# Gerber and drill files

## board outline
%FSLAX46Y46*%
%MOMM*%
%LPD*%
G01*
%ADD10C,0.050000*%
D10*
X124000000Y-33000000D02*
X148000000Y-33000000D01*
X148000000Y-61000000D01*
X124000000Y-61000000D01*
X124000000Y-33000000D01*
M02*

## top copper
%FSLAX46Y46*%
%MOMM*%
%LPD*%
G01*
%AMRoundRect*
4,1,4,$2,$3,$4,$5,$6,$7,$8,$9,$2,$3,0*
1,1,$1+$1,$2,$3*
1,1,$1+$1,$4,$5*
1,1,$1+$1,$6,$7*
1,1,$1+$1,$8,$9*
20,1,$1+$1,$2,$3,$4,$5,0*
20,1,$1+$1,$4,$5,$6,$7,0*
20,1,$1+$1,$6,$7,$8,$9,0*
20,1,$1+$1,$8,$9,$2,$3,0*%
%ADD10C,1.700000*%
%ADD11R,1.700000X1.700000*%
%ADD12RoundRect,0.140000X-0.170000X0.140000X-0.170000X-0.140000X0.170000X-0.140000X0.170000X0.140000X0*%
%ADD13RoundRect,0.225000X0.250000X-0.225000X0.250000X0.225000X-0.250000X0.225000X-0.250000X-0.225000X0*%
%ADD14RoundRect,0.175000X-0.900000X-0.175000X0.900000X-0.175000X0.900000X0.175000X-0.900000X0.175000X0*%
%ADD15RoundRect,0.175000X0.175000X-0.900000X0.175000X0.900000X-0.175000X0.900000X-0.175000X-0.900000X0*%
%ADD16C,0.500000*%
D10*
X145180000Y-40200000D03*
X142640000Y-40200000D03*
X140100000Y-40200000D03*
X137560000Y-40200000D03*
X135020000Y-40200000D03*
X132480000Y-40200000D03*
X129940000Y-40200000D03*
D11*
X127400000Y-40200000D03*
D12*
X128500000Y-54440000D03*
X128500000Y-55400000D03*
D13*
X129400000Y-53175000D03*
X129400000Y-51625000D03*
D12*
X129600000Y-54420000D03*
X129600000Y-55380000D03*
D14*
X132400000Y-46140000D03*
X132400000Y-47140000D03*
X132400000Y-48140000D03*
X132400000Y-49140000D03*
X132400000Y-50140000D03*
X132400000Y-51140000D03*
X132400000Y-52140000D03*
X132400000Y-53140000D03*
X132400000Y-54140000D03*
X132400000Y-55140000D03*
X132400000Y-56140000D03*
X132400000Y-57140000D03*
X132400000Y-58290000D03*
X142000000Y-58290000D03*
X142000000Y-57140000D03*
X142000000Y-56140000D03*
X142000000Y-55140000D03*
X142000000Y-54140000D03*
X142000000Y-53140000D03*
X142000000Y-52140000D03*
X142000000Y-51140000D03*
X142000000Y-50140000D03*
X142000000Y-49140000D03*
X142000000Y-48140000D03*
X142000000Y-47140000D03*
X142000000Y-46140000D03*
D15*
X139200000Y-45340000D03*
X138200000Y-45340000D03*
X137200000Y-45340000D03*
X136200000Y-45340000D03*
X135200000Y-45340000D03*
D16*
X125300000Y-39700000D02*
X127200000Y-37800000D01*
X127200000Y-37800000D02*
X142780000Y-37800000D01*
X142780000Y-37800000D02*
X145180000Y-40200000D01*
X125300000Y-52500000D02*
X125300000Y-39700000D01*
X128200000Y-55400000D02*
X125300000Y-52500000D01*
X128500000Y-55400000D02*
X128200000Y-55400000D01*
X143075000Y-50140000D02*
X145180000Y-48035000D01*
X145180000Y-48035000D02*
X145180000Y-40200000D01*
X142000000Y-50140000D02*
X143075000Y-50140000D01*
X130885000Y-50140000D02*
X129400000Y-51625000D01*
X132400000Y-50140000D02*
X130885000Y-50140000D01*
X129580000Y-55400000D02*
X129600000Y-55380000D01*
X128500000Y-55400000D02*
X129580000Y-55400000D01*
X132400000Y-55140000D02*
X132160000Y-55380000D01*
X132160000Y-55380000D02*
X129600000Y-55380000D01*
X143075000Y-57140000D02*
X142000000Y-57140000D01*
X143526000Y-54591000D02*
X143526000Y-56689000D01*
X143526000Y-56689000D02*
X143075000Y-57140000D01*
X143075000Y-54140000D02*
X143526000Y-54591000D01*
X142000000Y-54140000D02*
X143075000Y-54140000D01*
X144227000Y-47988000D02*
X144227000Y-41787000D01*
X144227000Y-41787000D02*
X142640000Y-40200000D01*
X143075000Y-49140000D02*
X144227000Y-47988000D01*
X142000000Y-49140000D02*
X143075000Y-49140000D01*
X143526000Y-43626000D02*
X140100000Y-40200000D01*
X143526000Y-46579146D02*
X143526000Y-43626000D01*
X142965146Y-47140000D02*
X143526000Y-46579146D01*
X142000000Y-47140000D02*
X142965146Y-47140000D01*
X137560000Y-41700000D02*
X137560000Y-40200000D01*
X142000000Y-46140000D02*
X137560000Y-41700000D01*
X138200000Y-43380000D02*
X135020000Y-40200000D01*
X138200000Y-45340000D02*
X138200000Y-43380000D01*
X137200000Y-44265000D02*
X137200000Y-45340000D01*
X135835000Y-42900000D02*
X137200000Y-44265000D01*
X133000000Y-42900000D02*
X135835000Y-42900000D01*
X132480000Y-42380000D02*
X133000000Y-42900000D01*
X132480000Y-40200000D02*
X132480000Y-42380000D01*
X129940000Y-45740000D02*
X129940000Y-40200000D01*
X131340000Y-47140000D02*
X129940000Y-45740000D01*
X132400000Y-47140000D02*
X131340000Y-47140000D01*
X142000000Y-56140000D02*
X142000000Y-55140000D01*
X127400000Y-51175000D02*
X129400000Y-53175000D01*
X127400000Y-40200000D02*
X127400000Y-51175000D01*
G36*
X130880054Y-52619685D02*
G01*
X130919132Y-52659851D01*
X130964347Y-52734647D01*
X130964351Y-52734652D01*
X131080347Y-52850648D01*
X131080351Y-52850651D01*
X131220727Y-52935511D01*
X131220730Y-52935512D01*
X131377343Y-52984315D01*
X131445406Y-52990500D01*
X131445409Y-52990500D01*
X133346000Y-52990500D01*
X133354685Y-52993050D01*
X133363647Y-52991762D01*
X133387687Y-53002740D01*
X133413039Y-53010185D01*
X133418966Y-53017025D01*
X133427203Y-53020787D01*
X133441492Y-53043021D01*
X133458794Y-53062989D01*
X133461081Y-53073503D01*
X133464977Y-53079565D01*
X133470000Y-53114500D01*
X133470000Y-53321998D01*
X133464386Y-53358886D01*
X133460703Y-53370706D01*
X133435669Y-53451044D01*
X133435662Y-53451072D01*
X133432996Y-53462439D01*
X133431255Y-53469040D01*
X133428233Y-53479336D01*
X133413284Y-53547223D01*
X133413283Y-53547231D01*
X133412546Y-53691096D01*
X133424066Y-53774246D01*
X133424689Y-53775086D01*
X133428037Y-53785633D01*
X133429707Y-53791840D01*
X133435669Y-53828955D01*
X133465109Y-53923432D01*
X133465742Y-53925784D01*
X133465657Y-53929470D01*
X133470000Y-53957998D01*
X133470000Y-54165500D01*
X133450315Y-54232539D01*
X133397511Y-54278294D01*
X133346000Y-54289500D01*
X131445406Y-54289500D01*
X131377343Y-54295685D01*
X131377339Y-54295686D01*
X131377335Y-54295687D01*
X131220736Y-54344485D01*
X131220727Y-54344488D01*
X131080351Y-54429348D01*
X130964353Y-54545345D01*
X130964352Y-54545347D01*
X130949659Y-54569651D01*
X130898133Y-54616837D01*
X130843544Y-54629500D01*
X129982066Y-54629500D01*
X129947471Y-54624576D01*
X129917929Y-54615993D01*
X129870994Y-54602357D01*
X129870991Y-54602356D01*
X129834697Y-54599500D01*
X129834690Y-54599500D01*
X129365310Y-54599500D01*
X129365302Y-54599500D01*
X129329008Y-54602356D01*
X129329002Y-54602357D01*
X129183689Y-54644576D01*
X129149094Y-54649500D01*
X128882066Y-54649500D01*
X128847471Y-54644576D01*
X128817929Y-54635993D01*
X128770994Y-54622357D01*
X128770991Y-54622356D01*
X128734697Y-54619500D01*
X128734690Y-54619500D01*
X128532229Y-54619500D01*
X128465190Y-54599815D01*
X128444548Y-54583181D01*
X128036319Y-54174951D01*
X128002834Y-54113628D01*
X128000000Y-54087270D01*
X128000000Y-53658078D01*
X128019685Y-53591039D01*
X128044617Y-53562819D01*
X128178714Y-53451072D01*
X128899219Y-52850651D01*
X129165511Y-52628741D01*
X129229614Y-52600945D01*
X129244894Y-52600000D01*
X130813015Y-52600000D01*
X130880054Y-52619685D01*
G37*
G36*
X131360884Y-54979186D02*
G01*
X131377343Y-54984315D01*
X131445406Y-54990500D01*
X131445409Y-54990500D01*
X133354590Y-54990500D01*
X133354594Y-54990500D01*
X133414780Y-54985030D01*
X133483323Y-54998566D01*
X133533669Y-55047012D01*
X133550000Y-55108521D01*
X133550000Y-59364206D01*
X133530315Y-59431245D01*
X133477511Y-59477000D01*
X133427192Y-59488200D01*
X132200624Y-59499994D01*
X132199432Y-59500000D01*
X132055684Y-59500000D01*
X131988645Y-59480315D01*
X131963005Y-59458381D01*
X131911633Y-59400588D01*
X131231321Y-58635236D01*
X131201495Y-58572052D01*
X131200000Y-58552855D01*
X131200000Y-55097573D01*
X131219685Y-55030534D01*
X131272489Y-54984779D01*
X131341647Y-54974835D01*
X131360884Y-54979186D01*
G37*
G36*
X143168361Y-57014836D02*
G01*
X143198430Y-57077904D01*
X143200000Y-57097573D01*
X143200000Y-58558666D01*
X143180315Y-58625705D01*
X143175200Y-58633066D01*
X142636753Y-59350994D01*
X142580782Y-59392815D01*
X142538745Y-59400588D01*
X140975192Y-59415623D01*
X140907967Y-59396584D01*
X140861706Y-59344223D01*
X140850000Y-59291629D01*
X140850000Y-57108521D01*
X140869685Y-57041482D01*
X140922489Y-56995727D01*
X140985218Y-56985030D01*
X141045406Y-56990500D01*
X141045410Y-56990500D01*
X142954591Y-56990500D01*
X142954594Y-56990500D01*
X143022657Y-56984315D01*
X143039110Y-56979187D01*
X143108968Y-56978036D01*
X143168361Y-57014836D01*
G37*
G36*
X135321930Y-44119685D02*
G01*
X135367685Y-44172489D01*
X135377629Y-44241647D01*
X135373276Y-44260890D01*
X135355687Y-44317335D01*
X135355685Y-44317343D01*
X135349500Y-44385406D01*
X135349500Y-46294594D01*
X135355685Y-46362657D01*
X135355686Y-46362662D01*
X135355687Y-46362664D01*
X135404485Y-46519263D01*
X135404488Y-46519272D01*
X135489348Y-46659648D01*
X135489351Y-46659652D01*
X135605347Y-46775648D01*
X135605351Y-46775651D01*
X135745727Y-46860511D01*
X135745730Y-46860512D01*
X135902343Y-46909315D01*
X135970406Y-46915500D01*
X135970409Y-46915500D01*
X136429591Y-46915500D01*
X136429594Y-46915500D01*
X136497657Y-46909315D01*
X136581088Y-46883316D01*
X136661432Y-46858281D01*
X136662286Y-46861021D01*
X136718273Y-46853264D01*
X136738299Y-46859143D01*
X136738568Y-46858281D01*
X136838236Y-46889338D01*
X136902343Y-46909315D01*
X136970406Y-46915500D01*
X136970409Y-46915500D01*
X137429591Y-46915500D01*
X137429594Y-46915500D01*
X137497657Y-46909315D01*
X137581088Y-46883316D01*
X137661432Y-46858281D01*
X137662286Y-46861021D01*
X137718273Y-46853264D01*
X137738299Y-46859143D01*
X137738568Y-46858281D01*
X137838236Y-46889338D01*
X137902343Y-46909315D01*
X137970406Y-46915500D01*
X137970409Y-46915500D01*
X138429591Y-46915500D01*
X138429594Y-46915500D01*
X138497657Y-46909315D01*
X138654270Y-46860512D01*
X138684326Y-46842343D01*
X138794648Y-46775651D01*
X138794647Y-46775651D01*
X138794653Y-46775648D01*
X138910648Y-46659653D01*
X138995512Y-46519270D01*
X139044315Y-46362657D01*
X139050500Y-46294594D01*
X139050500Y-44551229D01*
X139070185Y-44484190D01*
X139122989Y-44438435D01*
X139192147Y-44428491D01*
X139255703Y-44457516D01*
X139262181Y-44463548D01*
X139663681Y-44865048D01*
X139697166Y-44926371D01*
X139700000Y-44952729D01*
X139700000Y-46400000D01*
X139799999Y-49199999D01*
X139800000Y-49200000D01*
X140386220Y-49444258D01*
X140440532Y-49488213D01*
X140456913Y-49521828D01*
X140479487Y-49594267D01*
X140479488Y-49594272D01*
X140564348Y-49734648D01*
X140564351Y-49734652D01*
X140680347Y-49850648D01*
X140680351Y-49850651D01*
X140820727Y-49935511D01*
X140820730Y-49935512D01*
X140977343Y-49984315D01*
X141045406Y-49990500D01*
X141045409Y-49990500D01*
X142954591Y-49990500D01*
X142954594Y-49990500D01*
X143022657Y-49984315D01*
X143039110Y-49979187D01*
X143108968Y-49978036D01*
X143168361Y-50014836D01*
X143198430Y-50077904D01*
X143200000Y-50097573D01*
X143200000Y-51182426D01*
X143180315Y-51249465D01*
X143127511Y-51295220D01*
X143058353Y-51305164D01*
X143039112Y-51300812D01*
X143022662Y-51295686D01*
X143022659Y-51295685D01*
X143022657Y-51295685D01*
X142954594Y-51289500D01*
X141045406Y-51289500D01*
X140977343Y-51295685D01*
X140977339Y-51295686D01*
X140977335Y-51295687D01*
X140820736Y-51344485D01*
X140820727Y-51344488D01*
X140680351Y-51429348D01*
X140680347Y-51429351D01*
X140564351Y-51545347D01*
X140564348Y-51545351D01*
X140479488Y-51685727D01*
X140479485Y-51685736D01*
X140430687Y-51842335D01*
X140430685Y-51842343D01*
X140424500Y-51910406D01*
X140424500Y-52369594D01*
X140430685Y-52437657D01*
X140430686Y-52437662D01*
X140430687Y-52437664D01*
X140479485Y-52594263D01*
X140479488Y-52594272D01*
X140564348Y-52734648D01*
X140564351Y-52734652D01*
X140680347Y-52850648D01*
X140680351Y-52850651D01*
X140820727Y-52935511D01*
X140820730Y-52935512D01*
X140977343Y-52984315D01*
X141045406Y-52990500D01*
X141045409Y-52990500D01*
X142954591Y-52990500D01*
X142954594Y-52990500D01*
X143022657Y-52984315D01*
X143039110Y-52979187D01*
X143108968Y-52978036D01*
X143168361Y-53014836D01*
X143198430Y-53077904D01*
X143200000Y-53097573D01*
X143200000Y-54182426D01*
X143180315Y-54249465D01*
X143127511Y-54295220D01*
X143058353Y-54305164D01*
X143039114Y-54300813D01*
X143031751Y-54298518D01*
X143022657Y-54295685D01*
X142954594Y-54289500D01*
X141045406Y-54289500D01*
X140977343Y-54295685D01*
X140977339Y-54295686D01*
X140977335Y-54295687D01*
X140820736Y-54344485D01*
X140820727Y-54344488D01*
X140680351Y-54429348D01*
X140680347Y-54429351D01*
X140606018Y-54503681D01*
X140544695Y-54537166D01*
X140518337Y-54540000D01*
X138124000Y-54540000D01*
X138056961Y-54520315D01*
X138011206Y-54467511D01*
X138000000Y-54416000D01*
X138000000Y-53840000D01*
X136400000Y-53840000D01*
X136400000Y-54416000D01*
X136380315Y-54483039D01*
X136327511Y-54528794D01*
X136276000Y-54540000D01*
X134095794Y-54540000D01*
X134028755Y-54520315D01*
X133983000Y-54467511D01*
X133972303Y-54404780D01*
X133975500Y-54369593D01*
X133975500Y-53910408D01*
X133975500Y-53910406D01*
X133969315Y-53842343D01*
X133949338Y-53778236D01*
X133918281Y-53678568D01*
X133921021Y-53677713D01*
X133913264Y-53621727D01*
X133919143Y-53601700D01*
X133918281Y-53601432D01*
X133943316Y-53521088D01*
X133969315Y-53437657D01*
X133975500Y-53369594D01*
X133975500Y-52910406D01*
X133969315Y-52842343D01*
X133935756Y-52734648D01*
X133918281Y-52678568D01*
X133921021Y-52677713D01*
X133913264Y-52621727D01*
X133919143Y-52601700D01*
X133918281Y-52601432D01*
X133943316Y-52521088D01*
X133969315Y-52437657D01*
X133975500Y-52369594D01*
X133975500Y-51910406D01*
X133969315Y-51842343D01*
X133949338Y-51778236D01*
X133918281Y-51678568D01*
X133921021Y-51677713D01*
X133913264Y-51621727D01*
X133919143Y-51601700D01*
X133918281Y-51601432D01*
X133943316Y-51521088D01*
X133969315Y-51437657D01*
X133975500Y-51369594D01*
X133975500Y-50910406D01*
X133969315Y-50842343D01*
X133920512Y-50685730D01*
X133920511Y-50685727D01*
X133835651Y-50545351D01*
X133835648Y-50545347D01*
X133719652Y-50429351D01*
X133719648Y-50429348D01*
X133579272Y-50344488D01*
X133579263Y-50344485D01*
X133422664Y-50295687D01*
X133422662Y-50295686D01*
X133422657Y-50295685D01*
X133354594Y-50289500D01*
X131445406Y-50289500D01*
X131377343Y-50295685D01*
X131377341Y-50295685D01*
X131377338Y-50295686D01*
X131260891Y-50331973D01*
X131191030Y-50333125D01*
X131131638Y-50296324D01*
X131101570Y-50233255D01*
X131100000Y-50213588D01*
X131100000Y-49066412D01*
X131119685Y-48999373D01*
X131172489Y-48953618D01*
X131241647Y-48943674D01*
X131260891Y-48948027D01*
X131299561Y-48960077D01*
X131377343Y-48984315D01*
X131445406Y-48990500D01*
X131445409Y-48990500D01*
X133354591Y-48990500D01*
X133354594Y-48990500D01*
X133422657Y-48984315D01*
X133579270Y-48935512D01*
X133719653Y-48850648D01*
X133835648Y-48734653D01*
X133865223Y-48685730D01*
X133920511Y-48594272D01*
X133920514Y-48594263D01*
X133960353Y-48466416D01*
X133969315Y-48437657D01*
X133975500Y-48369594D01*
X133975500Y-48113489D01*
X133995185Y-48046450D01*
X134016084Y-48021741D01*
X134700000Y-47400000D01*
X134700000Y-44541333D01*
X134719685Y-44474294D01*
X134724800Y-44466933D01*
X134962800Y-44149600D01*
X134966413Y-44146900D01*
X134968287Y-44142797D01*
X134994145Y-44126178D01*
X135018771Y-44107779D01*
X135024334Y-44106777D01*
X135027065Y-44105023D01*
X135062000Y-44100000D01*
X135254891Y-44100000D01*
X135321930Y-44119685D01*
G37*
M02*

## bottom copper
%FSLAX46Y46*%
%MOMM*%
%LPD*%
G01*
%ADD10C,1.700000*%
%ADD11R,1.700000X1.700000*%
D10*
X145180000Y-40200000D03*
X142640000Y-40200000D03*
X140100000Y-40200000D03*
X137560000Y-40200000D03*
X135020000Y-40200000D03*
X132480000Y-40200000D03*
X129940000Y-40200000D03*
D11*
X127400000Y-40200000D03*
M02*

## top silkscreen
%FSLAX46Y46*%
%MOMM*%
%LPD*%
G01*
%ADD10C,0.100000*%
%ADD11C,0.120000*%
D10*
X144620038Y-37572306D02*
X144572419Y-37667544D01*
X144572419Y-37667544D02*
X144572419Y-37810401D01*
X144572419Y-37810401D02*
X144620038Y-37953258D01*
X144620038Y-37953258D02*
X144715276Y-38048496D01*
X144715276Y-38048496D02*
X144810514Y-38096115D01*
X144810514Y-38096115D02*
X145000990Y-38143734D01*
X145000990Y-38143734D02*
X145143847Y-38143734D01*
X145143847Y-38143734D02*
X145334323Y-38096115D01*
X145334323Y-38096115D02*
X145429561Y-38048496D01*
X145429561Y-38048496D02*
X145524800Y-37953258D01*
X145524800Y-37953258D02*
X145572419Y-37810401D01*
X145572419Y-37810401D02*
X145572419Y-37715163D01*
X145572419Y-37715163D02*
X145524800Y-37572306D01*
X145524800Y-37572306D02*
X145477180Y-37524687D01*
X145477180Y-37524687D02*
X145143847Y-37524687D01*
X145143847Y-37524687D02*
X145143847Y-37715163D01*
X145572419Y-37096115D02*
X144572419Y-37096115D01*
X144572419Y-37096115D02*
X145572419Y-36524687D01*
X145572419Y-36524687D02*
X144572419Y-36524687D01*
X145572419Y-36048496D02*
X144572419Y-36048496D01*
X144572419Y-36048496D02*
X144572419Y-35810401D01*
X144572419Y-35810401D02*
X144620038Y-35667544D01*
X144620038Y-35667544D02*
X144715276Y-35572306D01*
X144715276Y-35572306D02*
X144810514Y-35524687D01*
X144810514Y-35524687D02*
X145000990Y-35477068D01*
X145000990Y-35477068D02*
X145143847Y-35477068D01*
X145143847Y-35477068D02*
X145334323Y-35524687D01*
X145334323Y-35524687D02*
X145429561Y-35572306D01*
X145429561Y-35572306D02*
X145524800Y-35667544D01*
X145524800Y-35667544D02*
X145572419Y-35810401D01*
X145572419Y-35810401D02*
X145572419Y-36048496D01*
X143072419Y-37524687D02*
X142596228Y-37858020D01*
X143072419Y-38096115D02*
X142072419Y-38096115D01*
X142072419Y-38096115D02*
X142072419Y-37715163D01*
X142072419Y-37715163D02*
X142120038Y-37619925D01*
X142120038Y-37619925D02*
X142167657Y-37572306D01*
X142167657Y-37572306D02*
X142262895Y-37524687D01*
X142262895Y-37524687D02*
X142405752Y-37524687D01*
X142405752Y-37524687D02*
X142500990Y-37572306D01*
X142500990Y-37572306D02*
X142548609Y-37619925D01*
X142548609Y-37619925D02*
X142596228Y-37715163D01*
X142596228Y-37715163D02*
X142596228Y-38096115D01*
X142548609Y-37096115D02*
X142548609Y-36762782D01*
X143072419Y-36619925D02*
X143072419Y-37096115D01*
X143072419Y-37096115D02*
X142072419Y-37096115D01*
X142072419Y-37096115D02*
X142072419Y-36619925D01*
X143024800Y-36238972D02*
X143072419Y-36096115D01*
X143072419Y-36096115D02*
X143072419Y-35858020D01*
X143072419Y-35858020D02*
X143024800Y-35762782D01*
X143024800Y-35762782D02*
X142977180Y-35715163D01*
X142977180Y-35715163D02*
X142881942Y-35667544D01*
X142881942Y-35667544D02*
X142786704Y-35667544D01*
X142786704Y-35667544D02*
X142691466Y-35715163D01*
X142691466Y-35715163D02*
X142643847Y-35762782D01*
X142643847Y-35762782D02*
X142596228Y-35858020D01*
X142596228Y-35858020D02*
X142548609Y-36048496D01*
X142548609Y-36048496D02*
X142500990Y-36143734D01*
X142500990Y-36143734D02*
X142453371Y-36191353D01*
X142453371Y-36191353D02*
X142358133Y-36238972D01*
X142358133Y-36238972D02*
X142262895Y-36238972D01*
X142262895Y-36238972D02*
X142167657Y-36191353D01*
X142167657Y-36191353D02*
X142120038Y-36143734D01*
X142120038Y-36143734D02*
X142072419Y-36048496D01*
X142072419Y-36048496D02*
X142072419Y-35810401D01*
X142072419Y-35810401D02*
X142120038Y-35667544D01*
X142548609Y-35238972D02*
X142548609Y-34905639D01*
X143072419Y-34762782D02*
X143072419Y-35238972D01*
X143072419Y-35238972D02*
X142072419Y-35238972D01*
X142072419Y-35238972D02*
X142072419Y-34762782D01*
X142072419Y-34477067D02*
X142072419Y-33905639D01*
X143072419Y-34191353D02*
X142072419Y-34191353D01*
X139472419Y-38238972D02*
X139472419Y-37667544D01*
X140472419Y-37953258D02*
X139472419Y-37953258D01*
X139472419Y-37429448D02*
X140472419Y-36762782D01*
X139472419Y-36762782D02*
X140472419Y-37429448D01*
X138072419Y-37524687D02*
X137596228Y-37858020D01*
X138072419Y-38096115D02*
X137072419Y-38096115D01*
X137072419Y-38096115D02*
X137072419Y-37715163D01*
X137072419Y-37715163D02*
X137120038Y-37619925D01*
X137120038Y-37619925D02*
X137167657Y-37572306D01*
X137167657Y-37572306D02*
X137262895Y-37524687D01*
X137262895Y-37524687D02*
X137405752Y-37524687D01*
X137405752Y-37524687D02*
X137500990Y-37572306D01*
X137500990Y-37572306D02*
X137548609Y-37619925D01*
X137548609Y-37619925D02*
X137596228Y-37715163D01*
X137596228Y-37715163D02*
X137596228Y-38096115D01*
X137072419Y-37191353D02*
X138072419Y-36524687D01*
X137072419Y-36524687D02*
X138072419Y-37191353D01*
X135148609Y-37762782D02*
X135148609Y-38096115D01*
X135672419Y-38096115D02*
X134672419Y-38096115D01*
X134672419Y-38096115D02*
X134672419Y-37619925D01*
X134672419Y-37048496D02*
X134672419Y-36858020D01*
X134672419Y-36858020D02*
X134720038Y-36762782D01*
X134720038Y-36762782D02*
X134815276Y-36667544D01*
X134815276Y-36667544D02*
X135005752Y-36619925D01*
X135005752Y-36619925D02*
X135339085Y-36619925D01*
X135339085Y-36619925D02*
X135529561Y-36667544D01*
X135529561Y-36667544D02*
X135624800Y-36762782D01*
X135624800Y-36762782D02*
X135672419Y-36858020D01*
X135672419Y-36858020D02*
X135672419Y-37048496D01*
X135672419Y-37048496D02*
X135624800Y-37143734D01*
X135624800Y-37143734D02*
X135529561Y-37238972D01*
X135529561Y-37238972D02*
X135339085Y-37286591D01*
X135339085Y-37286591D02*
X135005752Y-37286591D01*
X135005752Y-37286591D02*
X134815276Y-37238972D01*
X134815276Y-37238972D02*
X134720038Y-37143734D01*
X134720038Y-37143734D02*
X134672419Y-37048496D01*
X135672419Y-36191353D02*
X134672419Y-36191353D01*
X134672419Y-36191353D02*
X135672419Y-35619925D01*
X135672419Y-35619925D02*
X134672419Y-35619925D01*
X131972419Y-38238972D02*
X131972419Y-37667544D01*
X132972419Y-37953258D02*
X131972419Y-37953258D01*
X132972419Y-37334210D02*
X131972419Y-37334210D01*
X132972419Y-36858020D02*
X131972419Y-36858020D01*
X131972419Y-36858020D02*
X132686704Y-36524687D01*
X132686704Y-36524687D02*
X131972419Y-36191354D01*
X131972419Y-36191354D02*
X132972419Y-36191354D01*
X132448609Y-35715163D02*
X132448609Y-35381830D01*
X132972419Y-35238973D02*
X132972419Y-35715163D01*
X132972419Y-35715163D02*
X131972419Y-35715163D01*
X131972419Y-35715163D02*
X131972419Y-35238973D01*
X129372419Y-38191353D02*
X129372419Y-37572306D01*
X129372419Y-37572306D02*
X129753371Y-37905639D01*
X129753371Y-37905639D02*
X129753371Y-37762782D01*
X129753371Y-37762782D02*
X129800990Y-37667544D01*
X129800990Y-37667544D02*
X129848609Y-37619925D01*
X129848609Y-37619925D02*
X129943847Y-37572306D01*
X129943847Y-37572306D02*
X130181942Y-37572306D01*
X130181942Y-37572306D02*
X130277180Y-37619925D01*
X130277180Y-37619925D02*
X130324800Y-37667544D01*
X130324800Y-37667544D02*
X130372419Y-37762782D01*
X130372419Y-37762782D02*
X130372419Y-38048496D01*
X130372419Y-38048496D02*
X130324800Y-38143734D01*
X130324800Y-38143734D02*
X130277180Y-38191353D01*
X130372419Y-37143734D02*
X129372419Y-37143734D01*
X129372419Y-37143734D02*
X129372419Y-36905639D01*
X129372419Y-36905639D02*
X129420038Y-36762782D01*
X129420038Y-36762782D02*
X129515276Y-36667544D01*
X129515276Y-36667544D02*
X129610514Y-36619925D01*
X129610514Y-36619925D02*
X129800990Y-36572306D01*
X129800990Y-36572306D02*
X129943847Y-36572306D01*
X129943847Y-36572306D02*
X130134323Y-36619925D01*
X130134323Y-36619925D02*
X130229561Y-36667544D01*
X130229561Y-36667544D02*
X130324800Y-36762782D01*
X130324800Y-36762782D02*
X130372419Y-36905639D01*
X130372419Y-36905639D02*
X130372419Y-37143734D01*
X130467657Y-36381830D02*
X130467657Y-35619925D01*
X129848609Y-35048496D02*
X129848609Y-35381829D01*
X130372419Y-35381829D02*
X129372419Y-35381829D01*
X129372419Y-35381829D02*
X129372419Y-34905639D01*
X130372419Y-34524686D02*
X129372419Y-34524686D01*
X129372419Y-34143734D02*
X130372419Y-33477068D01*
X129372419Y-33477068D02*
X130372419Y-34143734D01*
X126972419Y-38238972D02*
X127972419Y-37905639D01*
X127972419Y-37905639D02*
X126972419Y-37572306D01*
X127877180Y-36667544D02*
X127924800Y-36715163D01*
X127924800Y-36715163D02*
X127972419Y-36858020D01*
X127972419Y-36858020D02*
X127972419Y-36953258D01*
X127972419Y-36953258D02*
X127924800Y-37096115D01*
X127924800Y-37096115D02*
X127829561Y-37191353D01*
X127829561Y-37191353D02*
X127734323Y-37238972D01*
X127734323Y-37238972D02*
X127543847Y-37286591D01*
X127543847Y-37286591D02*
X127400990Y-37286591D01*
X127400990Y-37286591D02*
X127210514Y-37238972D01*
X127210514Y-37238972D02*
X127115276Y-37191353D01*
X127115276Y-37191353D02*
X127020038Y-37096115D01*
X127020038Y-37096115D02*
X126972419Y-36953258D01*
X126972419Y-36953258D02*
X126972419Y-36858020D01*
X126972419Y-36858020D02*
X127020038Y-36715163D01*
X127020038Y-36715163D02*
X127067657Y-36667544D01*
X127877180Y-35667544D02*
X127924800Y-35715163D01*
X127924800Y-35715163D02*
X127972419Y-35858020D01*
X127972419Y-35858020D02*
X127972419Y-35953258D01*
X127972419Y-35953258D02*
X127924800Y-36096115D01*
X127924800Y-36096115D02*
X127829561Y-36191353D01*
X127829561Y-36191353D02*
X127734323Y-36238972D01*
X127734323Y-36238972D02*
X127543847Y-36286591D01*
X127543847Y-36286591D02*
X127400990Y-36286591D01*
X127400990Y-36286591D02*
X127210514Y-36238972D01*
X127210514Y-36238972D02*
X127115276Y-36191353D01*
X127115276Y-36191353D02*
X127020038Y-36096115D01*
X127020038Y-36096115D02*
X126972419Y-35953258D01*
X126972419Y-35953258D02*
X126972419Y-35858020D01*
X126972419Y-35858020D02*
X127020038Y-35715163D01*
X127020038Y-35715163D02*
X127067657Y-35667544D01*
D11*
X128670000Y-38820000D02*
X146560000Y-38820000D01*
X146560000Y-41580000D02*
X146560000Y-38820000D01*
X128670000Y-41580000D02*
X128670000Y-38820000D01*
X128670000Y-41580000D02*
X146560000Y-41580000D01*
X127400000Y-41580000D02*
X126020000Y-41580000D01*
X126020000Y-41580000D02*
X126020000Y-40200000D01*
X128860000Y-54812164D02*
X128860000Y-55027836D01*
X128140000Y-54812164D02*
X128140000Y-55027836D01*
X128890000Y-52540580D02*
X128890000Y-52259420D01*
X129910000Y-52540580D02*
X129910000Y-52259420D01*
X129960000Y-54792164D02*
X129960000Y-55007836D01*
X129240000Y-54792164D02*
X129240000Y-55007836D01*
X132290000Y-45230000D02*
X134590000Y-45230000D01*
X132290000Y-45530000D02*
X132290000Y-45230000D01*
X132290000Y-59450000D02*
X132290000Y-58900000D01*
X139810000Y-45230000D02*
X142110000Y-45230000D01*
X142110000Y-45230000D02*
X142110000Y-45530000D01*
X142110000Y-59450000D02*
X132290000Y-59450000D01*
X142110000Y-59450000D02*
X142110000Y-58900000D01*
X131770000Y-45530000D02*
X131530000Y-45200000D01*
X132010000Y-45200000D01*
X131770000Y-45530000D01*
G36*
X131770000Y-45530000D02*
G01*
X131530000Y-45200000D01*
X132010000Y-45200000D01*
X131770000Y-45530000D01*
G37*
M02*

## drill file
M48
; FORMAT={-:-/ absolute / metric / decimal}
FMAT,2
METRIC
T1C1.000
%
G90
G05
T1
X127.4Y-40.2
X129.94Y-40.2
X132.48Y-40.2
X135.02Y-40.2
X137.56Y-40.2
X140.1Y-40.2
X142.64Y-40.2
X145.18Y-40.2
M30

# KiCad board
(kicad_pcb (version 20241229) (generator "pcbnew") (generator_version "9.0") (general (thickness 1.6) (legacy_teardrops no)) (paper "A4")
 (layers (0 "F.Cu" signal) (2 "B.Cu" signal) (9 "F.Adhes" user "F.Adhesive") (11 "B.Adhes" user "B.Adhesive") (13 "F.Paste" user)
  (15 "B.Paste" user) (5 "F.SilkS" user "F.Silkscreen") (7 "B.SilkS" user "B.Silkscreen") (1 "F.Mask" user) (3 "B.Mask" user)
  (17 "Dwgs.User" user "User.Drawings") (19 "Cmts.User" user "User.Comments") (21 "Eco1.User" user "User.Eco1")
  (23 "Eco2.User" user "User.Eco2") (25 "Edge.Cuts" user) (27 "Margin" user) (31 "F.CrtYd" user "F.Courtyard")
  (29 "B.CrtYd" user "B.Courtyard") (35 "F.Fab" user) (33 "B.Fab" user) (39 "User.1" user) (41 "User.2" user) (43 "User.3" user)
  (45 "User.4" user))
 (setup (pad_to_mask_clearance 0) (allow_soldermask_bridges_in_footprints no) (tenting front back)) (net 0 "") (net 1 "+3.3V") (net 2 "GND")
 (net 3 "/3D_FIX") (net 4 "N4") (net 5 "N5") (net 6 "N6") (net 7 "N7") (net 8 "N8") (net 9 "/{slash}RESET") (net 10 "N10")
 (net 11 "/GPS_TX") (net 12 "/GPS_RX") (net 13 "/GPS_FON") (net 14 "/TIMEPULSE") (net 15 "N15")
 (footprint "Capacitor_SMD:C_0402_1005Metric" (layer "F.Cu") (at 128.5 54.92 -90)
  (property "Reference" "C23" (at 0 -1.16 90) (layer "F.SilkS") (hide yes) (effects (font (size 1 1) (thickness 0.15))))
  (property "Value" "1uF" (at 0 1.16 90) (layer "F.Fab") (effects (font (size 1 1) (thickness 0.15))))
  (fp_line (start -0.107836 0.36) (end 0.107836 0.36) (stroke (width 0.12) (type solid)) (layer "F.SilkS"))
  (fp_line (start -0.107836 -0.36) (end 0.107836 -0.36) (stroke (width 0.12) (type solid)) (layer "F.SilkS"))
  (pad "1" smd roundrect (at -0.48 0 270) (size 0.56 0.62) (layers "F.Cu" "F.Mask" "F.Paste") (roundrect_rratio 0.25) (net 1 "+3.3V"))
  (pad "2" smd roundrect (at 0.48 0 270) (size 0.56 0.62) (layers "F.Cu" "F.Mask" "F.Paste") (roundrect_rratio 0.25) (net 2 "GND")))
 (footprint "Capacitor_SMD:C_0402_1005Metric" (layer "F.Cu") (at 129.6 54.9 -90)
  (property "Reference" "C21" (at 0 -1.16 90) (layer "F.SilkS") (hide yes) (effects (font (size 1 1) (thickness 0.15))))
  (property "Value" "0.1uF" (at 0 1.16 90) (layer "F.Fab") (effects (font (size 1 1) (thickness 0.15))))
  (fp_line (start -0.107836 0.36) (end 0.107836 0.36) (stroke (width 0.12) (type solid)) (layer "F.SilkS"))
  (fp_line (start -0.107836 -0.36) (end 0.107836 -0.36) (stroke (width 0.12) (type solid)) (layer "F.SilkS"))
  (pad "1" smd roundrect (at -0.48 0 270) (size 0.56 0.62) (layers "F.Cu" "F.Mask" "F.Paste") (roundrect_rratio 0.25) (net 1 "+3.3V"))
  (pad "2" smd roundrect (at 0.48 0 270) (size 0.56 0.62) (layers "F.Cu" "F.Mask" "F.Paste") (roundrect_rratio 0.25) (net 2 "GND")))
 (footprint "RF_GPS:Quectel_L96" (layer "F.Cu") (at 137.2 52.34)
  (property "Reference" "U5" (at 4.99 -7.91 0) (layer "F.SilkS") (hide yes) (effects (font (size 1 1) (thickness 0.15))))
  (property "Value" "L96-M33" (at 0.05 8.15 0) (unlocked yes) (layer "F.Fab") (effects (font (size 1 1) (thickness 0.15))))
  (fp_line (start -4.91 -7.11) (end -2.61 -7.11) (stroke (width 0.12) (type default)) (layer "F.SilkS"))
  (fp_line (start -4.91 -6.81) (end -4.91 -7.11) (stroke (width 0.12) (type default)) (layer "F.SilkS"))
  (fp_line (start -4.91 7.11) (end -4.91 6.56) (stroke (width 0.12) (type default)) (layer "F.SilkS"))
  (fp_line (start 2.61 -7.11) (end 4.91 -7.11) (stroke (width 0.12) (type default)) (layer "F.SilkS"))
  (fp_line (start 4.91 -7.11) (end 4.91 -6.81) (stroke (width 0.12) (type default)) (layer "F.SilkS"))
  (fp_line (start 4.91 7.11) (end -4.91 7.11) (stroke (width 0.12) (type default)) (layer "F.SilkS"))
  (fp_line (start 4.91 7.11) (end 4.91 6.56) (stroke (width 0.12) (type default)) (layer "F.SilkS"))
  (fp_poly
   (pts (xy -5.43 -6.81) (xy -5.67 -7.14) (xy -5.19 -7.14) (xy -5.43 -6.81)) (stroke (width 0.12) (type solid)) (fill yes) (layer "F.SilkS"))
  (pad "1" smd roundrect (at -4.8 -6.2) (size 2.15 0.7) (layers "F.Cu" "F.Mask" "F.Paste") (roundrect_rratio 0.25) (thermal_bridge_angle 45))
  (pad "2" smd roundrect (at -4.8 -5.2) (size 2.15 0.7) (layers "F.Cu" "F.Mask" "F.Paste") (roundrect_rratio 0.25) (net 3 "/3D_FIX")
   (thermal_bridge_angle 45))
  (pad "3" smd roundrect (at -4.8 -4.2) (size 2.15 0.7) (layers "F.Cu" "F.Mask" "F.Paste") (roundrect_rratio 0.25) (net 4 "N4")
   (thermal_bridge_angle 45))
  (pad "4" smd roundrect (at -4.8 -3.2) (size 2.15 0.7) (layers "F.Cu" "F.Mask" "F.Paste") (roundrect_rratio 0.25) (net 2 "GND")
   (thermal_bridge_angle 45))
  (pad "5" smd roundrect (at -4.8 -2.2) (size 2.15 0.7) (layers "F.Cu" "F.Mask" "F.Paste") (roundrect_rratio 0.25) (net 2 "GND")
   (thermal_bridge_angle 45))
  (pad "6" smd roundrect (at -4.8 -1.2) (size 2.15 0.7) (layers "F.Cu" "F.Mask" "F.Paste") (roundrect_rratio 0.25) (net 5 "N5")
   (thermal_bridge_angle 45))
  (pad "7" smd roundrect (at -4.8 -0.2) (size 2.15 0.7) (layers "F.Cu" "F.Mask" "F.Paste") (roundrect_rratio 0.25) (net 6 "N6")
   (thermal_bridge_angle 45))
  (pad "8" smd roundrect (at -4.8 0.8) (size 2.15 0.7) (layers "F.Cu" "F.Mask" "F.Paste") (roundrect_rratio 0.25) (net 1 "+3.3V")
   (thermal_bridge_angle 45))
  (pad "9" smd roundrect (at -4.8 1.8) (size 2.15 0.7) (layers "F.Cu" "F.Mask" "F.Paste") (roundrect_rratio 0.25) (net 1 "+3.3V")
   (thermal_bridge_angle 45))
  (pad "10" smd roundrect (at -4.8 2.8) (size 2.15 0.7) (layers "F.Cu" "F.Mask" "F.Paste") (roundrect_rratio 0.25) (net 2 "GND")
   (thermal_bridge_angle 45))
  (pad "11" smd roundrect (at -4.8 3.8) (size 2.15 0.7) (layers "F.Cu" "F.Mask" "F.Paste") (roundrect_rratio 0.25) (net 2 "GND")
   (thermal_bridge_angle 45))
  (pad "12" smd roundrect (at -4.8 4.8) (size 2.15 0.7) (layers "F.Cu" "F.Mask" "F.Paste") (roundrect_rratio 0.25) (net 2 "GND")
   (thermal_bridge_angle 45))
  (pad "13" smd roundrect (at -4.8 5.95) (size 2.15 0.7) (layers "F.Cu" "F.Mask" "F.Paste") (roundrect_rratio 0.25) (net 2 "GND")
   (thermal_bridge_angle 45))
  (pad "14" smd roundrect (at 4.8 5.95) (size 2.15 0.7) (layers "F.Cu" "F.Mask" "F.Paste") (roundrect_rratio 0.25) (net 2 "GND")
   (thermal_bridge_angle 45))
  (pad "15" smd roundrect (at 4.8 4.8) (size 2.15 0.7) (layers "F.Cu" "F.Mask" "F.Paste") (roundrect_rratio 0.25) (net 2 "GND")
   (thermal_bridge_angle 45))
  (pad "16" smd roundrect (at 4.8 3.8) (size 2.15 0.7) (layers "F.Cu" "F.Mask" "F.Paste") (roundrect_rratio 0.25) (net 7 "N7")
   (thermal_bridge_angle 45))
  (pad "17" smd roundrect (at 4.8 2.8) (size 2.15 0.7) (layers "F.Cu" "F.Mask" "F.Paste") (roundrect_rratio 0.25) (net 7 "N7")
   (thermal_bridge_angle 45))
  (pad "18" smd roundrect (at 4.8 1.8) (size 2.15 0.7) (layers "F.Cu" "F.Mask" "F.Paste") (roundrect_rratio 0.25) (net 2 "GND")
   (thermal_bridge_angle 45))
  (pad "19" smd roundrect (at 4.8 0.8) (size 2.15 0.7) (layers "F.Cu" "F.Mask" "F.Paste") (roundrect_rratio 0.25) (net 2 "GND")
   (thermal_bridge_angle 45))
  (pad "20" smd roundrect (at 4.8 -0.2) (size 2.15 0.7) (layers "F.Cu" "F.Mask" "F.Paste") (roundrect_rratio 0.25) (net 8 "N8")
   (thermal_bridge_angle 45))
  (pad "21" smd roundrect (at 4.8 -1.2) (size 2.15 0.7) (layers "F.Cu" "F.Mask" "F.Paste") (roundrect_rratio 0.25) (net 2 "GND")
   (thermal_bridge_angle 45))
  (pad "22" smd roundrect (at 4.8 -2.2) (size 2.15 0.7) (layers "F.Cu" "F.Mask" "F.Paste") (roundrect_rratio 0.25) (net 2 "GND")
   (thermal_bridge_angle 45))
  (pad "23" smd roundrect (at 4.8 -3.2) (size 2.15 0.7) (layers "F.Cu" "F.Mask" "F.Paste") (roundrect_rratio 0.25) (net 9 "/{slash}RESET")
   (thermal_bridge_angle 45))
  (pad "24" smd roundrect (at 4.8 -4.2) (size 2.15 0.7) (layers "F.Cu" "F.Mask" "F.Paste") (roundrect_rratio 0.25) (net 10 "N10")
   (thermal_bridge_angle 45))
  (pad "25" smd roundrect (at 4.8 -5.2) (size 2.15 0.7) (layers "F.Cu" "F.Mask" "F.Paste") (roundrect_rratio 0.25) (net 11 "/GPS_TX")
   (thermal_bridge_angle 45))
  (pad "26" smd roundrect (at 4.8 -6.2) (size 2.15 0.7) (layers "F.Cu" "F.Mask" "F.Paste") (roundrect_rratio 0.25) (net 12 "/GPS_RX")
   (thermal_bridge_angle 45))
  (pad "27" smd roundrect (at 2 -7 90) (size 2.15 0.7) (layers "F.Cu" "F.Mask" "F.Paste") (roundrect_rratio 0.25) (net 2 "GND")
   (thermal_bridge_angle 45))
  (pad "28" smd roundrect (at 1 -7 90) (size 2.15 0.7) (layers "F.Cu" "F.Mask" "F.Paste") (roundrect_rratio 0.25) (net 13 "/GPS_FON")
   (thermal_bridge_angle 45))
  (pad "29" smd roundrect (at 0 -7 90) (size 2.15 0.7) (layers "F.Cu" "F.Mask" "F.Paste") (roundrect_rratio 0.25) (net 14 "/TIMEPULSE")
   (thermal_bridge_angle 45))
  (pad "30" smd roundrect (at -1 -7 90) (size 2.15 0.7) (layers "F.Cu" "F.Mask" "F.Paste") (roundrect_rratio 0.25) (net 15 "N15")
   (thermal_bridge_angle 45))
  (pad "31" smd roundrect (at -2 -7 90) (size 2.15 0.7) (layers "F.Cu" "F.Mask" "F.Paste") (roundrect_rratio 0.25) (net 2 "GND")
   (thermal_bridge_angle 45))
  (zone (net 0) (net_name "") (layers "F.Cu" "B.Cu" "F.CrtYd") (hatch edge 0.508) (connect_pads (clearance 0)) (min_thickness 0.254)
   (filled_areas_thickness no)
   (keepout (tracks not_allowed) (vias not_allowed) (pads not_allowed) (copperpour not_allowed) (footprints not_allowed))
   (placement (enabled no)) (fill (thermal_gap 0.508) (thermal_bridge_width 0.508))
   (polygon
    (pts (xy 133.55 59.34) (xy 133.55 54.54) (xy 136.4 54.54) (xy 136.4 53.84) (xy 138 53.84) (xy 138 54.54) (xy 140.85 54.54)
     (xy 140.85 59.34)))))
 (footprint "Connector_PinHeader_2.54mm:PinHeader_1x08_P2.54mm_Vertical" (layer "F.Cu") (at 127.4 40.2 90)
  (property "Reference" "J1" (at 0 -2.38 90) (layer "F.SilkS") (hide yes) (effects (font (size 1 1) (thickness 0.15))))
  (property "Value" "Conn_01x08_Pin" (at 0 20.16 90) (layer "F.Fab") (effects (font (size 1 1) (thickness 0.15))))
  (fp_line (start -1.38 -1.38) (end 0 -1.38) (stroke (width 0.12) (type solid)) (layer "F.SilkS"))
  (fp_line (start -1.38 0) (end -1.38 -1.38) (stroke (width 0.12) (type solid)) (layer "F.SilkS"))
  (fp_line (start 1.38 1.27) (end 1.38 19.16) (stroke (width 0.12) (type solid)) (layer "F.SilkS"))
  (fp_line (start -1.38 1.27) (end 1.38 1.27) (stroke (width 0.12) (type solid)) (layer "F.SilkS"))
  (fp_line (start -1.38 1.27) (end -1.38 19.16) (stroke (width 0.12) (type solid)) (layer "F.SilkS"))
  (fp_line (start -1.38 19.16) (end 1.38 19.16) (stroke (width 0.12) (type solid)) (layer "F.SilkS"))
  (pad "1" thru_hole rect (at 0 0 90) (size 1.7 1.7) (drill 1) (layers "*.Cu" "*.Mask") (remove_unused_layers no) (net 1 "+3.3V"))
  (pad "2" thru_hole circle (at 0 2.54 90) (size 1.7 1.7) (drill 1) (layers "*.Cu" "*.Mask") (remove_unused_layers no) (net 3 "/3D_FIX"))
  (pad "3" thru_hole circle (at 0 5.08 90) (size 1.7 1.7) (drill 1) (layers "*.Cu" "*.Mask") (remove_unused_layers no) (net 14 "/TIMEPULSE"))
  (pad "4" thru_hole circle (at 0 7.62 90) (size 1.7 1.7) (drill 1) (layers "*.Cu" "*.Mask") (remove_unused_layers no) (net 13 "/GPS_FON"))
  (pad "5" thru_hole circle (at 0 10.16 90) (size 1.7 1.7) (drill 1) (layers "*.Cu" "*.Mask") (remove_unused_layers no) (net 12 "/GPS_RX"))
  (pad "6" thru_hole circle (at 0 12.7 90) (size 1.7 1.7) (drill 1) (layers "*.Cu" "*.Mask") (remove_unused_layers no) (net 11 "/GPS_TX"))
  (pad "7" thru_hole circle (at 0 15.24 90) (size 1.7 1.7) (drill 1) (layers "*.Cu" "*.Mask") (remove_unused_layers no)
   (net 9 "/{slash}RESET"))
  (pad "8" thru_hole circle (at 0 17.78 90) (size 1.7 1.7) (drill 1) (layers "*.Cu" "*.Mask") (remove_unused_layers no) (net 2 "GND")))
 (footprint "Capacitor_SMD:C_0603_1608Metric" (layer "F.Cu") (at 129.4 52.4 90)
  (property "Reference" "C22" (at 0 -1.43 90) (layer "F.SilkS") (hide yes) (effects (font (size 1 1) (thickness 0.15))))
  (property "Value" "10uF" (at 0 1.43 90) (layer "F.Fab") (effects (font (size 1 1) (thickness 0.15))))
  (fp_line (start -0.14058 -0.51) (end 0.14058 -0.51) (stroke (width 0.12) (type solid)) (layer "F.SilkS"))
  (fp_line (start -0.14058 0.51) (end 0.14058 0.51) (stroke (width 0.12) (type solid)) (layer "F.SilkS"))
  (pad "1" smd roundrect (at -0.775 0 90) (size 0.9 0.95) (layers "F.Cu" "F.Mask" "F.Paste") (roundrect_rratio 0.25) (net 1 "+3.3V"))
  (pad "2" smd roundrect (at 0.775 0 90) (size 0.9 0.95) (layers "F.Cu" "F.Mask" "F.Paste") (roundrect_rratio 0.25) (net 2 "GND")))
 (gr_rect (start 124 33) (end 148 61) (stroke (width 0.05) (type default)) (fill no) (layer "Edge.Cuts"))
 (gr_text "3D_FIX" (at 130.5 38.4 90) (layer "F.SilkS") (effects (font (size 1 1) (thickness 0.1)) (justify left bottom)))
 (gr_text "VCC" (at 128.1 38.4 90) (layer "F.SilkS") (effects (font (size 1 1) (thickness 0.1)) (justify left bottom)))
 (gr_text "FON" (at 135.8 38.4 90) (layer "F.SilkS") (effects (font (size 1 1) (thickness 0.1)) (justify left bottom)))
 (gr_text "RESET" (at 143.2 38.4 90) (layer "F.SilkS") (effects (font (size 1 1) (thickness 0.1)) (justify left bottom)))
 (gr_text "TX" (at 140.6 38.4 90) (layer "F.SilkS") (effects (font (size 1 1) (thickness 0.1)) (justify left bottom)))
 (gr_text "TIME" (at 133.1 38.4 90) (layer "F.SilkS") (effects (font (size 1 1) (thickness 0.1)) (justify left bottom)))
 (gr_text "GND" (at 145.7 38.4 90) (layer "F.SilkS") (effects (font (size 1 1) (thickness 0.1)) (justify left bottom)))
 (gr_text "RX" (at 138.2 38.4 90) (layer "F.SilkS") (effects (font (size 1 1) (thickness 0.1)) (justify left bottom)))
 (segment (start 143.075 50.14) (end 145.18 48.035) (width 0.5) (layer "F.Cu") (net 2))
 (segment (start 143.075 54.14) (end 143.526 54.591) (width 0.5) (layer "F.Cu") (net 2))
 (segment (start 143.075 57.14) (end 142 57.14) (width 0.5) (layer "F.Cu") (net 2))
 (segment (start 130.885 50.14) (end 129.4 51.625) (width 0.5) (layer "F.Cu") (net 2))
 (segment (start 128.5 55.4) (end 128.2 55.4) (width 0.5) (layer "F.Cu") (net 2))
 (segment (start 125.3 39.7) (end 127.2 37.8) (width 0.5) (layer "F.Cu") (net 2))
 (segment (start 142 50.14) (end 143.075 50.14) (width 0.5) (layer "F.Cu") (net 2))
 (segment (start 128.5 55.4) (end 129.58 55.4) (width 0.5) (layer "F.Cu") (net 2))
 (segment (start 128.2 55.4) (end 125.3 52.5) (width 0.5) (layer "F.Cu") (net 2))
 (segment (start 132.4 50.14) (end 130.885 50.14) (width 0.5) (layer "F.Cu") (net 2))
 (segment (start 129.58 55.4) (end 129.6 55.38) (width 0.5) (layer "F.Cu") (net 2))
 (segment (start 142.78 37.8) (end 145.18 40.2) (width 0.5) (layer "F.Cu") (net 2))
 (segment (start 142 54.14) (end 143.075 54.14) (width 0.5) (layer "F.Cu") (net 2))
 (segment (start 143.526 56.689) (end 143.075 57.14) (width 0.5) (layer "F.Cu") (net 2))
 (segment (start 145.18 48.035) (end 145.18 40.2) (width 0.5) (layer "F.Cu") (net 2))
 (segment (start 125.3 52.5) (end 125.3 39.7) (width 0.5) (layer "F.Cu") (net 2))
 (segment (start 127.2 37.8) (end 142.78 37.8) (width 0.5) (layer "F.Cu") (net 2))
 (segment (start 143.526 54.591) (end 143.526 56.689) (width 0.5) (layer "F.Cu") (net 2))
 (segment (start 132.16 55.38) (end 129.6 55.38) (width 0.5) (layer "F.Cu") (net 2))
 (segment (start 132.4 55.14) (end 132.16 55.38) (width 0.5) (layer "F.Cu") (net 2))
 (segment (start 127.4 51.175) (end 129.4 53.175) (width 0.5) (layer "F.Cu") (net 1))
 (segment (start 127.4 40.2) (end 127.4 51.175) (width 0.5) (layer "F.Cu") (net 1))
 (segment (start 138.2 45.34) (end 138.2 43.38) (width 0.5) (layer "F.Cu") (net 13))
 (segment (start 138.2 43.38) (end 135.02 40.2) (width 0.5) (layer "F.Cu") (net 13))
 (segment (start 143.526 46.579146) (end 143.526 43.626) (width 0.5) (layer "F.Cu") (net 11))
 (segment (start 143.526 43.626) (end 140.1 40.2) (width 0.5) (layer "F.Cu") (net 11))
 (segment (start 142 47.14) (end 142.965146 47.14) (width 0.5) (layer "F.Cu") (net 11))
 (segment (start 142.965146 47.14) (end 143.526 46.579146) (width 0.5) (layer "F.Cu") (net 11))
 (segment (start 143.075 49.14) (end 144.227 47.988) (width 0.5) (layer "F.Cu") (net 9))
 (segment (start 144.227 47.988) (end 144.227 41.787) (width 0.5) (layer "F.Cu") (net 9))
 (segment (start 142 49.14) (end 143.075 49.14) (width 0.5) (layer "F.Cu") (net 9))
 (segment (start 144.227 41.787) (end 142.64 40.2) (width 0.5) (layer "F.Cu") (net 9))
 (segment (start 129.94 45.74) (end 129.94 40.2) (width 0.5) (layer "F.Cu") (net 3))
 (segment (start 132.4 47.14) (end 131.34 47.14) (width 0.5) (layer "F.Cu") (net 3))
 (segment (start 131.34 47.14) (end 129.94 45.74) (width 0.5) (layer "F.Cu") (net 3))
 (segment (start 142 46.14) (end 137.56 41.7) (width 0.5) (layer "F.Cu") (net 12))
 (segment (start 137.56 41.7) (end 137.56 40.2) (width 0.5) (layer "F.Cu") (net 12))
 (segment (start 133 42.9) (end 135.835 42.9) (width 0.5) (layer "F.Cu") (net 14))
 (segment (start 132.48 42.38) (end 133 42.9) (width 0.5) (layer "F.Cu") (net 14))
 (segment (start 132.48 40.2) (end 132.48 42.38) (width 0.5) (layer "F.Cu") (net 14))
 (segment (start 137.2 44.265) (end 137.2 45.34) (width 0.5) (layer "F.Cu") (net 14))
 (segment (start 135.835 42.9) (end 137.2 44.265) (width 0.5) (layer "F.Cu") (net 14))
 (segment (start 142 56.14) (end 142 55.14) (width 0.5) (layer "F.Cu") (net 7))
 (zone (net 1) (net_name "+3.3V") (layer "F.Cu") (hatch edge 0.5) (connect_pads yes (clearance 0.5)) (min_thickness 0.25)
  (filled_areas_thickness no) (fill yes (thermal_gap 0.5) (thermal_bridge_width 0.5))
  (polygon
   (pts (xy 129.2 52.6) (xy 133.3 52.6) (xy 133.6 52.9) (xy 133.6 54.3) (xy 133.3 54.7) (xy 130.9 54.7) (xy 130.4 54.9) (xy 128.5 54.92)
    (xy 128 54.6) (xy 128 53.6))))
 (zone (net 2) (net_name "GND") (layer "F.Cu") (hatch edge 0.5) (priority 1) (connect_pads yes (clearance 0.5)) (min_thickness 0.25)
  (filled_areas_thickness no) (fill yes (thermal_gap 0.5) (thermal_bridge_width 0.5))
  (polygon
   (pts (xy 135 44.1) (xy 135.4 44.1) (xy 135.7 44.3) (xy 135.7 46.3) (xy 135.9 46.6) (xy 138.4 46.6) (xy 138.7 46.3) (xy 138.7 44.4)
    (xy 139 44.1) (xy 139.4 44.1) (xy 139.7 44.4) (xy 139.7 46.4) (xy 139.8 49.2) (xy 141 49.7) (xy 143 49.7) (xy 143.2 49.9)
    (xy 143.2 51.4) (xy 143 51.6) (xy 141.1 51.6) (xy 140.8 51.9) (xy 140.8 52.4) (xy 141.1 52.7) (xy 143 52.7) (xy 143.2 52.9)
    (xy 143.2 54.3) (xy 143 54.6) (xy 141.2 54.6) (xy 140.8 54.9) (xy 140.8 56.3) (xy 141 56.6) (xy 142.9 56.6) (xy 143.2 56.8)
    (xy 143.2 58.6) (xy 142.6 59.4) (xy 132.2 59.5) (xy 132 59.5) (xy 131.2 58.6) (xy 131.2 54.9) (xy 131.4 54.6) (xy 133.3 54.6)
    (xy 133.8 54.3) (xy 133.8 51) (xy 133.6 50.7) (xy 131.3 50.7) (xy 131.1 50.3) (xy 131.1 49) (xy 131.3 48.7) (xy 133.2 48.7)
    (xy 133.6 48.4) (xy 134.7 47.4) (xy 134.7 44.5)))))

